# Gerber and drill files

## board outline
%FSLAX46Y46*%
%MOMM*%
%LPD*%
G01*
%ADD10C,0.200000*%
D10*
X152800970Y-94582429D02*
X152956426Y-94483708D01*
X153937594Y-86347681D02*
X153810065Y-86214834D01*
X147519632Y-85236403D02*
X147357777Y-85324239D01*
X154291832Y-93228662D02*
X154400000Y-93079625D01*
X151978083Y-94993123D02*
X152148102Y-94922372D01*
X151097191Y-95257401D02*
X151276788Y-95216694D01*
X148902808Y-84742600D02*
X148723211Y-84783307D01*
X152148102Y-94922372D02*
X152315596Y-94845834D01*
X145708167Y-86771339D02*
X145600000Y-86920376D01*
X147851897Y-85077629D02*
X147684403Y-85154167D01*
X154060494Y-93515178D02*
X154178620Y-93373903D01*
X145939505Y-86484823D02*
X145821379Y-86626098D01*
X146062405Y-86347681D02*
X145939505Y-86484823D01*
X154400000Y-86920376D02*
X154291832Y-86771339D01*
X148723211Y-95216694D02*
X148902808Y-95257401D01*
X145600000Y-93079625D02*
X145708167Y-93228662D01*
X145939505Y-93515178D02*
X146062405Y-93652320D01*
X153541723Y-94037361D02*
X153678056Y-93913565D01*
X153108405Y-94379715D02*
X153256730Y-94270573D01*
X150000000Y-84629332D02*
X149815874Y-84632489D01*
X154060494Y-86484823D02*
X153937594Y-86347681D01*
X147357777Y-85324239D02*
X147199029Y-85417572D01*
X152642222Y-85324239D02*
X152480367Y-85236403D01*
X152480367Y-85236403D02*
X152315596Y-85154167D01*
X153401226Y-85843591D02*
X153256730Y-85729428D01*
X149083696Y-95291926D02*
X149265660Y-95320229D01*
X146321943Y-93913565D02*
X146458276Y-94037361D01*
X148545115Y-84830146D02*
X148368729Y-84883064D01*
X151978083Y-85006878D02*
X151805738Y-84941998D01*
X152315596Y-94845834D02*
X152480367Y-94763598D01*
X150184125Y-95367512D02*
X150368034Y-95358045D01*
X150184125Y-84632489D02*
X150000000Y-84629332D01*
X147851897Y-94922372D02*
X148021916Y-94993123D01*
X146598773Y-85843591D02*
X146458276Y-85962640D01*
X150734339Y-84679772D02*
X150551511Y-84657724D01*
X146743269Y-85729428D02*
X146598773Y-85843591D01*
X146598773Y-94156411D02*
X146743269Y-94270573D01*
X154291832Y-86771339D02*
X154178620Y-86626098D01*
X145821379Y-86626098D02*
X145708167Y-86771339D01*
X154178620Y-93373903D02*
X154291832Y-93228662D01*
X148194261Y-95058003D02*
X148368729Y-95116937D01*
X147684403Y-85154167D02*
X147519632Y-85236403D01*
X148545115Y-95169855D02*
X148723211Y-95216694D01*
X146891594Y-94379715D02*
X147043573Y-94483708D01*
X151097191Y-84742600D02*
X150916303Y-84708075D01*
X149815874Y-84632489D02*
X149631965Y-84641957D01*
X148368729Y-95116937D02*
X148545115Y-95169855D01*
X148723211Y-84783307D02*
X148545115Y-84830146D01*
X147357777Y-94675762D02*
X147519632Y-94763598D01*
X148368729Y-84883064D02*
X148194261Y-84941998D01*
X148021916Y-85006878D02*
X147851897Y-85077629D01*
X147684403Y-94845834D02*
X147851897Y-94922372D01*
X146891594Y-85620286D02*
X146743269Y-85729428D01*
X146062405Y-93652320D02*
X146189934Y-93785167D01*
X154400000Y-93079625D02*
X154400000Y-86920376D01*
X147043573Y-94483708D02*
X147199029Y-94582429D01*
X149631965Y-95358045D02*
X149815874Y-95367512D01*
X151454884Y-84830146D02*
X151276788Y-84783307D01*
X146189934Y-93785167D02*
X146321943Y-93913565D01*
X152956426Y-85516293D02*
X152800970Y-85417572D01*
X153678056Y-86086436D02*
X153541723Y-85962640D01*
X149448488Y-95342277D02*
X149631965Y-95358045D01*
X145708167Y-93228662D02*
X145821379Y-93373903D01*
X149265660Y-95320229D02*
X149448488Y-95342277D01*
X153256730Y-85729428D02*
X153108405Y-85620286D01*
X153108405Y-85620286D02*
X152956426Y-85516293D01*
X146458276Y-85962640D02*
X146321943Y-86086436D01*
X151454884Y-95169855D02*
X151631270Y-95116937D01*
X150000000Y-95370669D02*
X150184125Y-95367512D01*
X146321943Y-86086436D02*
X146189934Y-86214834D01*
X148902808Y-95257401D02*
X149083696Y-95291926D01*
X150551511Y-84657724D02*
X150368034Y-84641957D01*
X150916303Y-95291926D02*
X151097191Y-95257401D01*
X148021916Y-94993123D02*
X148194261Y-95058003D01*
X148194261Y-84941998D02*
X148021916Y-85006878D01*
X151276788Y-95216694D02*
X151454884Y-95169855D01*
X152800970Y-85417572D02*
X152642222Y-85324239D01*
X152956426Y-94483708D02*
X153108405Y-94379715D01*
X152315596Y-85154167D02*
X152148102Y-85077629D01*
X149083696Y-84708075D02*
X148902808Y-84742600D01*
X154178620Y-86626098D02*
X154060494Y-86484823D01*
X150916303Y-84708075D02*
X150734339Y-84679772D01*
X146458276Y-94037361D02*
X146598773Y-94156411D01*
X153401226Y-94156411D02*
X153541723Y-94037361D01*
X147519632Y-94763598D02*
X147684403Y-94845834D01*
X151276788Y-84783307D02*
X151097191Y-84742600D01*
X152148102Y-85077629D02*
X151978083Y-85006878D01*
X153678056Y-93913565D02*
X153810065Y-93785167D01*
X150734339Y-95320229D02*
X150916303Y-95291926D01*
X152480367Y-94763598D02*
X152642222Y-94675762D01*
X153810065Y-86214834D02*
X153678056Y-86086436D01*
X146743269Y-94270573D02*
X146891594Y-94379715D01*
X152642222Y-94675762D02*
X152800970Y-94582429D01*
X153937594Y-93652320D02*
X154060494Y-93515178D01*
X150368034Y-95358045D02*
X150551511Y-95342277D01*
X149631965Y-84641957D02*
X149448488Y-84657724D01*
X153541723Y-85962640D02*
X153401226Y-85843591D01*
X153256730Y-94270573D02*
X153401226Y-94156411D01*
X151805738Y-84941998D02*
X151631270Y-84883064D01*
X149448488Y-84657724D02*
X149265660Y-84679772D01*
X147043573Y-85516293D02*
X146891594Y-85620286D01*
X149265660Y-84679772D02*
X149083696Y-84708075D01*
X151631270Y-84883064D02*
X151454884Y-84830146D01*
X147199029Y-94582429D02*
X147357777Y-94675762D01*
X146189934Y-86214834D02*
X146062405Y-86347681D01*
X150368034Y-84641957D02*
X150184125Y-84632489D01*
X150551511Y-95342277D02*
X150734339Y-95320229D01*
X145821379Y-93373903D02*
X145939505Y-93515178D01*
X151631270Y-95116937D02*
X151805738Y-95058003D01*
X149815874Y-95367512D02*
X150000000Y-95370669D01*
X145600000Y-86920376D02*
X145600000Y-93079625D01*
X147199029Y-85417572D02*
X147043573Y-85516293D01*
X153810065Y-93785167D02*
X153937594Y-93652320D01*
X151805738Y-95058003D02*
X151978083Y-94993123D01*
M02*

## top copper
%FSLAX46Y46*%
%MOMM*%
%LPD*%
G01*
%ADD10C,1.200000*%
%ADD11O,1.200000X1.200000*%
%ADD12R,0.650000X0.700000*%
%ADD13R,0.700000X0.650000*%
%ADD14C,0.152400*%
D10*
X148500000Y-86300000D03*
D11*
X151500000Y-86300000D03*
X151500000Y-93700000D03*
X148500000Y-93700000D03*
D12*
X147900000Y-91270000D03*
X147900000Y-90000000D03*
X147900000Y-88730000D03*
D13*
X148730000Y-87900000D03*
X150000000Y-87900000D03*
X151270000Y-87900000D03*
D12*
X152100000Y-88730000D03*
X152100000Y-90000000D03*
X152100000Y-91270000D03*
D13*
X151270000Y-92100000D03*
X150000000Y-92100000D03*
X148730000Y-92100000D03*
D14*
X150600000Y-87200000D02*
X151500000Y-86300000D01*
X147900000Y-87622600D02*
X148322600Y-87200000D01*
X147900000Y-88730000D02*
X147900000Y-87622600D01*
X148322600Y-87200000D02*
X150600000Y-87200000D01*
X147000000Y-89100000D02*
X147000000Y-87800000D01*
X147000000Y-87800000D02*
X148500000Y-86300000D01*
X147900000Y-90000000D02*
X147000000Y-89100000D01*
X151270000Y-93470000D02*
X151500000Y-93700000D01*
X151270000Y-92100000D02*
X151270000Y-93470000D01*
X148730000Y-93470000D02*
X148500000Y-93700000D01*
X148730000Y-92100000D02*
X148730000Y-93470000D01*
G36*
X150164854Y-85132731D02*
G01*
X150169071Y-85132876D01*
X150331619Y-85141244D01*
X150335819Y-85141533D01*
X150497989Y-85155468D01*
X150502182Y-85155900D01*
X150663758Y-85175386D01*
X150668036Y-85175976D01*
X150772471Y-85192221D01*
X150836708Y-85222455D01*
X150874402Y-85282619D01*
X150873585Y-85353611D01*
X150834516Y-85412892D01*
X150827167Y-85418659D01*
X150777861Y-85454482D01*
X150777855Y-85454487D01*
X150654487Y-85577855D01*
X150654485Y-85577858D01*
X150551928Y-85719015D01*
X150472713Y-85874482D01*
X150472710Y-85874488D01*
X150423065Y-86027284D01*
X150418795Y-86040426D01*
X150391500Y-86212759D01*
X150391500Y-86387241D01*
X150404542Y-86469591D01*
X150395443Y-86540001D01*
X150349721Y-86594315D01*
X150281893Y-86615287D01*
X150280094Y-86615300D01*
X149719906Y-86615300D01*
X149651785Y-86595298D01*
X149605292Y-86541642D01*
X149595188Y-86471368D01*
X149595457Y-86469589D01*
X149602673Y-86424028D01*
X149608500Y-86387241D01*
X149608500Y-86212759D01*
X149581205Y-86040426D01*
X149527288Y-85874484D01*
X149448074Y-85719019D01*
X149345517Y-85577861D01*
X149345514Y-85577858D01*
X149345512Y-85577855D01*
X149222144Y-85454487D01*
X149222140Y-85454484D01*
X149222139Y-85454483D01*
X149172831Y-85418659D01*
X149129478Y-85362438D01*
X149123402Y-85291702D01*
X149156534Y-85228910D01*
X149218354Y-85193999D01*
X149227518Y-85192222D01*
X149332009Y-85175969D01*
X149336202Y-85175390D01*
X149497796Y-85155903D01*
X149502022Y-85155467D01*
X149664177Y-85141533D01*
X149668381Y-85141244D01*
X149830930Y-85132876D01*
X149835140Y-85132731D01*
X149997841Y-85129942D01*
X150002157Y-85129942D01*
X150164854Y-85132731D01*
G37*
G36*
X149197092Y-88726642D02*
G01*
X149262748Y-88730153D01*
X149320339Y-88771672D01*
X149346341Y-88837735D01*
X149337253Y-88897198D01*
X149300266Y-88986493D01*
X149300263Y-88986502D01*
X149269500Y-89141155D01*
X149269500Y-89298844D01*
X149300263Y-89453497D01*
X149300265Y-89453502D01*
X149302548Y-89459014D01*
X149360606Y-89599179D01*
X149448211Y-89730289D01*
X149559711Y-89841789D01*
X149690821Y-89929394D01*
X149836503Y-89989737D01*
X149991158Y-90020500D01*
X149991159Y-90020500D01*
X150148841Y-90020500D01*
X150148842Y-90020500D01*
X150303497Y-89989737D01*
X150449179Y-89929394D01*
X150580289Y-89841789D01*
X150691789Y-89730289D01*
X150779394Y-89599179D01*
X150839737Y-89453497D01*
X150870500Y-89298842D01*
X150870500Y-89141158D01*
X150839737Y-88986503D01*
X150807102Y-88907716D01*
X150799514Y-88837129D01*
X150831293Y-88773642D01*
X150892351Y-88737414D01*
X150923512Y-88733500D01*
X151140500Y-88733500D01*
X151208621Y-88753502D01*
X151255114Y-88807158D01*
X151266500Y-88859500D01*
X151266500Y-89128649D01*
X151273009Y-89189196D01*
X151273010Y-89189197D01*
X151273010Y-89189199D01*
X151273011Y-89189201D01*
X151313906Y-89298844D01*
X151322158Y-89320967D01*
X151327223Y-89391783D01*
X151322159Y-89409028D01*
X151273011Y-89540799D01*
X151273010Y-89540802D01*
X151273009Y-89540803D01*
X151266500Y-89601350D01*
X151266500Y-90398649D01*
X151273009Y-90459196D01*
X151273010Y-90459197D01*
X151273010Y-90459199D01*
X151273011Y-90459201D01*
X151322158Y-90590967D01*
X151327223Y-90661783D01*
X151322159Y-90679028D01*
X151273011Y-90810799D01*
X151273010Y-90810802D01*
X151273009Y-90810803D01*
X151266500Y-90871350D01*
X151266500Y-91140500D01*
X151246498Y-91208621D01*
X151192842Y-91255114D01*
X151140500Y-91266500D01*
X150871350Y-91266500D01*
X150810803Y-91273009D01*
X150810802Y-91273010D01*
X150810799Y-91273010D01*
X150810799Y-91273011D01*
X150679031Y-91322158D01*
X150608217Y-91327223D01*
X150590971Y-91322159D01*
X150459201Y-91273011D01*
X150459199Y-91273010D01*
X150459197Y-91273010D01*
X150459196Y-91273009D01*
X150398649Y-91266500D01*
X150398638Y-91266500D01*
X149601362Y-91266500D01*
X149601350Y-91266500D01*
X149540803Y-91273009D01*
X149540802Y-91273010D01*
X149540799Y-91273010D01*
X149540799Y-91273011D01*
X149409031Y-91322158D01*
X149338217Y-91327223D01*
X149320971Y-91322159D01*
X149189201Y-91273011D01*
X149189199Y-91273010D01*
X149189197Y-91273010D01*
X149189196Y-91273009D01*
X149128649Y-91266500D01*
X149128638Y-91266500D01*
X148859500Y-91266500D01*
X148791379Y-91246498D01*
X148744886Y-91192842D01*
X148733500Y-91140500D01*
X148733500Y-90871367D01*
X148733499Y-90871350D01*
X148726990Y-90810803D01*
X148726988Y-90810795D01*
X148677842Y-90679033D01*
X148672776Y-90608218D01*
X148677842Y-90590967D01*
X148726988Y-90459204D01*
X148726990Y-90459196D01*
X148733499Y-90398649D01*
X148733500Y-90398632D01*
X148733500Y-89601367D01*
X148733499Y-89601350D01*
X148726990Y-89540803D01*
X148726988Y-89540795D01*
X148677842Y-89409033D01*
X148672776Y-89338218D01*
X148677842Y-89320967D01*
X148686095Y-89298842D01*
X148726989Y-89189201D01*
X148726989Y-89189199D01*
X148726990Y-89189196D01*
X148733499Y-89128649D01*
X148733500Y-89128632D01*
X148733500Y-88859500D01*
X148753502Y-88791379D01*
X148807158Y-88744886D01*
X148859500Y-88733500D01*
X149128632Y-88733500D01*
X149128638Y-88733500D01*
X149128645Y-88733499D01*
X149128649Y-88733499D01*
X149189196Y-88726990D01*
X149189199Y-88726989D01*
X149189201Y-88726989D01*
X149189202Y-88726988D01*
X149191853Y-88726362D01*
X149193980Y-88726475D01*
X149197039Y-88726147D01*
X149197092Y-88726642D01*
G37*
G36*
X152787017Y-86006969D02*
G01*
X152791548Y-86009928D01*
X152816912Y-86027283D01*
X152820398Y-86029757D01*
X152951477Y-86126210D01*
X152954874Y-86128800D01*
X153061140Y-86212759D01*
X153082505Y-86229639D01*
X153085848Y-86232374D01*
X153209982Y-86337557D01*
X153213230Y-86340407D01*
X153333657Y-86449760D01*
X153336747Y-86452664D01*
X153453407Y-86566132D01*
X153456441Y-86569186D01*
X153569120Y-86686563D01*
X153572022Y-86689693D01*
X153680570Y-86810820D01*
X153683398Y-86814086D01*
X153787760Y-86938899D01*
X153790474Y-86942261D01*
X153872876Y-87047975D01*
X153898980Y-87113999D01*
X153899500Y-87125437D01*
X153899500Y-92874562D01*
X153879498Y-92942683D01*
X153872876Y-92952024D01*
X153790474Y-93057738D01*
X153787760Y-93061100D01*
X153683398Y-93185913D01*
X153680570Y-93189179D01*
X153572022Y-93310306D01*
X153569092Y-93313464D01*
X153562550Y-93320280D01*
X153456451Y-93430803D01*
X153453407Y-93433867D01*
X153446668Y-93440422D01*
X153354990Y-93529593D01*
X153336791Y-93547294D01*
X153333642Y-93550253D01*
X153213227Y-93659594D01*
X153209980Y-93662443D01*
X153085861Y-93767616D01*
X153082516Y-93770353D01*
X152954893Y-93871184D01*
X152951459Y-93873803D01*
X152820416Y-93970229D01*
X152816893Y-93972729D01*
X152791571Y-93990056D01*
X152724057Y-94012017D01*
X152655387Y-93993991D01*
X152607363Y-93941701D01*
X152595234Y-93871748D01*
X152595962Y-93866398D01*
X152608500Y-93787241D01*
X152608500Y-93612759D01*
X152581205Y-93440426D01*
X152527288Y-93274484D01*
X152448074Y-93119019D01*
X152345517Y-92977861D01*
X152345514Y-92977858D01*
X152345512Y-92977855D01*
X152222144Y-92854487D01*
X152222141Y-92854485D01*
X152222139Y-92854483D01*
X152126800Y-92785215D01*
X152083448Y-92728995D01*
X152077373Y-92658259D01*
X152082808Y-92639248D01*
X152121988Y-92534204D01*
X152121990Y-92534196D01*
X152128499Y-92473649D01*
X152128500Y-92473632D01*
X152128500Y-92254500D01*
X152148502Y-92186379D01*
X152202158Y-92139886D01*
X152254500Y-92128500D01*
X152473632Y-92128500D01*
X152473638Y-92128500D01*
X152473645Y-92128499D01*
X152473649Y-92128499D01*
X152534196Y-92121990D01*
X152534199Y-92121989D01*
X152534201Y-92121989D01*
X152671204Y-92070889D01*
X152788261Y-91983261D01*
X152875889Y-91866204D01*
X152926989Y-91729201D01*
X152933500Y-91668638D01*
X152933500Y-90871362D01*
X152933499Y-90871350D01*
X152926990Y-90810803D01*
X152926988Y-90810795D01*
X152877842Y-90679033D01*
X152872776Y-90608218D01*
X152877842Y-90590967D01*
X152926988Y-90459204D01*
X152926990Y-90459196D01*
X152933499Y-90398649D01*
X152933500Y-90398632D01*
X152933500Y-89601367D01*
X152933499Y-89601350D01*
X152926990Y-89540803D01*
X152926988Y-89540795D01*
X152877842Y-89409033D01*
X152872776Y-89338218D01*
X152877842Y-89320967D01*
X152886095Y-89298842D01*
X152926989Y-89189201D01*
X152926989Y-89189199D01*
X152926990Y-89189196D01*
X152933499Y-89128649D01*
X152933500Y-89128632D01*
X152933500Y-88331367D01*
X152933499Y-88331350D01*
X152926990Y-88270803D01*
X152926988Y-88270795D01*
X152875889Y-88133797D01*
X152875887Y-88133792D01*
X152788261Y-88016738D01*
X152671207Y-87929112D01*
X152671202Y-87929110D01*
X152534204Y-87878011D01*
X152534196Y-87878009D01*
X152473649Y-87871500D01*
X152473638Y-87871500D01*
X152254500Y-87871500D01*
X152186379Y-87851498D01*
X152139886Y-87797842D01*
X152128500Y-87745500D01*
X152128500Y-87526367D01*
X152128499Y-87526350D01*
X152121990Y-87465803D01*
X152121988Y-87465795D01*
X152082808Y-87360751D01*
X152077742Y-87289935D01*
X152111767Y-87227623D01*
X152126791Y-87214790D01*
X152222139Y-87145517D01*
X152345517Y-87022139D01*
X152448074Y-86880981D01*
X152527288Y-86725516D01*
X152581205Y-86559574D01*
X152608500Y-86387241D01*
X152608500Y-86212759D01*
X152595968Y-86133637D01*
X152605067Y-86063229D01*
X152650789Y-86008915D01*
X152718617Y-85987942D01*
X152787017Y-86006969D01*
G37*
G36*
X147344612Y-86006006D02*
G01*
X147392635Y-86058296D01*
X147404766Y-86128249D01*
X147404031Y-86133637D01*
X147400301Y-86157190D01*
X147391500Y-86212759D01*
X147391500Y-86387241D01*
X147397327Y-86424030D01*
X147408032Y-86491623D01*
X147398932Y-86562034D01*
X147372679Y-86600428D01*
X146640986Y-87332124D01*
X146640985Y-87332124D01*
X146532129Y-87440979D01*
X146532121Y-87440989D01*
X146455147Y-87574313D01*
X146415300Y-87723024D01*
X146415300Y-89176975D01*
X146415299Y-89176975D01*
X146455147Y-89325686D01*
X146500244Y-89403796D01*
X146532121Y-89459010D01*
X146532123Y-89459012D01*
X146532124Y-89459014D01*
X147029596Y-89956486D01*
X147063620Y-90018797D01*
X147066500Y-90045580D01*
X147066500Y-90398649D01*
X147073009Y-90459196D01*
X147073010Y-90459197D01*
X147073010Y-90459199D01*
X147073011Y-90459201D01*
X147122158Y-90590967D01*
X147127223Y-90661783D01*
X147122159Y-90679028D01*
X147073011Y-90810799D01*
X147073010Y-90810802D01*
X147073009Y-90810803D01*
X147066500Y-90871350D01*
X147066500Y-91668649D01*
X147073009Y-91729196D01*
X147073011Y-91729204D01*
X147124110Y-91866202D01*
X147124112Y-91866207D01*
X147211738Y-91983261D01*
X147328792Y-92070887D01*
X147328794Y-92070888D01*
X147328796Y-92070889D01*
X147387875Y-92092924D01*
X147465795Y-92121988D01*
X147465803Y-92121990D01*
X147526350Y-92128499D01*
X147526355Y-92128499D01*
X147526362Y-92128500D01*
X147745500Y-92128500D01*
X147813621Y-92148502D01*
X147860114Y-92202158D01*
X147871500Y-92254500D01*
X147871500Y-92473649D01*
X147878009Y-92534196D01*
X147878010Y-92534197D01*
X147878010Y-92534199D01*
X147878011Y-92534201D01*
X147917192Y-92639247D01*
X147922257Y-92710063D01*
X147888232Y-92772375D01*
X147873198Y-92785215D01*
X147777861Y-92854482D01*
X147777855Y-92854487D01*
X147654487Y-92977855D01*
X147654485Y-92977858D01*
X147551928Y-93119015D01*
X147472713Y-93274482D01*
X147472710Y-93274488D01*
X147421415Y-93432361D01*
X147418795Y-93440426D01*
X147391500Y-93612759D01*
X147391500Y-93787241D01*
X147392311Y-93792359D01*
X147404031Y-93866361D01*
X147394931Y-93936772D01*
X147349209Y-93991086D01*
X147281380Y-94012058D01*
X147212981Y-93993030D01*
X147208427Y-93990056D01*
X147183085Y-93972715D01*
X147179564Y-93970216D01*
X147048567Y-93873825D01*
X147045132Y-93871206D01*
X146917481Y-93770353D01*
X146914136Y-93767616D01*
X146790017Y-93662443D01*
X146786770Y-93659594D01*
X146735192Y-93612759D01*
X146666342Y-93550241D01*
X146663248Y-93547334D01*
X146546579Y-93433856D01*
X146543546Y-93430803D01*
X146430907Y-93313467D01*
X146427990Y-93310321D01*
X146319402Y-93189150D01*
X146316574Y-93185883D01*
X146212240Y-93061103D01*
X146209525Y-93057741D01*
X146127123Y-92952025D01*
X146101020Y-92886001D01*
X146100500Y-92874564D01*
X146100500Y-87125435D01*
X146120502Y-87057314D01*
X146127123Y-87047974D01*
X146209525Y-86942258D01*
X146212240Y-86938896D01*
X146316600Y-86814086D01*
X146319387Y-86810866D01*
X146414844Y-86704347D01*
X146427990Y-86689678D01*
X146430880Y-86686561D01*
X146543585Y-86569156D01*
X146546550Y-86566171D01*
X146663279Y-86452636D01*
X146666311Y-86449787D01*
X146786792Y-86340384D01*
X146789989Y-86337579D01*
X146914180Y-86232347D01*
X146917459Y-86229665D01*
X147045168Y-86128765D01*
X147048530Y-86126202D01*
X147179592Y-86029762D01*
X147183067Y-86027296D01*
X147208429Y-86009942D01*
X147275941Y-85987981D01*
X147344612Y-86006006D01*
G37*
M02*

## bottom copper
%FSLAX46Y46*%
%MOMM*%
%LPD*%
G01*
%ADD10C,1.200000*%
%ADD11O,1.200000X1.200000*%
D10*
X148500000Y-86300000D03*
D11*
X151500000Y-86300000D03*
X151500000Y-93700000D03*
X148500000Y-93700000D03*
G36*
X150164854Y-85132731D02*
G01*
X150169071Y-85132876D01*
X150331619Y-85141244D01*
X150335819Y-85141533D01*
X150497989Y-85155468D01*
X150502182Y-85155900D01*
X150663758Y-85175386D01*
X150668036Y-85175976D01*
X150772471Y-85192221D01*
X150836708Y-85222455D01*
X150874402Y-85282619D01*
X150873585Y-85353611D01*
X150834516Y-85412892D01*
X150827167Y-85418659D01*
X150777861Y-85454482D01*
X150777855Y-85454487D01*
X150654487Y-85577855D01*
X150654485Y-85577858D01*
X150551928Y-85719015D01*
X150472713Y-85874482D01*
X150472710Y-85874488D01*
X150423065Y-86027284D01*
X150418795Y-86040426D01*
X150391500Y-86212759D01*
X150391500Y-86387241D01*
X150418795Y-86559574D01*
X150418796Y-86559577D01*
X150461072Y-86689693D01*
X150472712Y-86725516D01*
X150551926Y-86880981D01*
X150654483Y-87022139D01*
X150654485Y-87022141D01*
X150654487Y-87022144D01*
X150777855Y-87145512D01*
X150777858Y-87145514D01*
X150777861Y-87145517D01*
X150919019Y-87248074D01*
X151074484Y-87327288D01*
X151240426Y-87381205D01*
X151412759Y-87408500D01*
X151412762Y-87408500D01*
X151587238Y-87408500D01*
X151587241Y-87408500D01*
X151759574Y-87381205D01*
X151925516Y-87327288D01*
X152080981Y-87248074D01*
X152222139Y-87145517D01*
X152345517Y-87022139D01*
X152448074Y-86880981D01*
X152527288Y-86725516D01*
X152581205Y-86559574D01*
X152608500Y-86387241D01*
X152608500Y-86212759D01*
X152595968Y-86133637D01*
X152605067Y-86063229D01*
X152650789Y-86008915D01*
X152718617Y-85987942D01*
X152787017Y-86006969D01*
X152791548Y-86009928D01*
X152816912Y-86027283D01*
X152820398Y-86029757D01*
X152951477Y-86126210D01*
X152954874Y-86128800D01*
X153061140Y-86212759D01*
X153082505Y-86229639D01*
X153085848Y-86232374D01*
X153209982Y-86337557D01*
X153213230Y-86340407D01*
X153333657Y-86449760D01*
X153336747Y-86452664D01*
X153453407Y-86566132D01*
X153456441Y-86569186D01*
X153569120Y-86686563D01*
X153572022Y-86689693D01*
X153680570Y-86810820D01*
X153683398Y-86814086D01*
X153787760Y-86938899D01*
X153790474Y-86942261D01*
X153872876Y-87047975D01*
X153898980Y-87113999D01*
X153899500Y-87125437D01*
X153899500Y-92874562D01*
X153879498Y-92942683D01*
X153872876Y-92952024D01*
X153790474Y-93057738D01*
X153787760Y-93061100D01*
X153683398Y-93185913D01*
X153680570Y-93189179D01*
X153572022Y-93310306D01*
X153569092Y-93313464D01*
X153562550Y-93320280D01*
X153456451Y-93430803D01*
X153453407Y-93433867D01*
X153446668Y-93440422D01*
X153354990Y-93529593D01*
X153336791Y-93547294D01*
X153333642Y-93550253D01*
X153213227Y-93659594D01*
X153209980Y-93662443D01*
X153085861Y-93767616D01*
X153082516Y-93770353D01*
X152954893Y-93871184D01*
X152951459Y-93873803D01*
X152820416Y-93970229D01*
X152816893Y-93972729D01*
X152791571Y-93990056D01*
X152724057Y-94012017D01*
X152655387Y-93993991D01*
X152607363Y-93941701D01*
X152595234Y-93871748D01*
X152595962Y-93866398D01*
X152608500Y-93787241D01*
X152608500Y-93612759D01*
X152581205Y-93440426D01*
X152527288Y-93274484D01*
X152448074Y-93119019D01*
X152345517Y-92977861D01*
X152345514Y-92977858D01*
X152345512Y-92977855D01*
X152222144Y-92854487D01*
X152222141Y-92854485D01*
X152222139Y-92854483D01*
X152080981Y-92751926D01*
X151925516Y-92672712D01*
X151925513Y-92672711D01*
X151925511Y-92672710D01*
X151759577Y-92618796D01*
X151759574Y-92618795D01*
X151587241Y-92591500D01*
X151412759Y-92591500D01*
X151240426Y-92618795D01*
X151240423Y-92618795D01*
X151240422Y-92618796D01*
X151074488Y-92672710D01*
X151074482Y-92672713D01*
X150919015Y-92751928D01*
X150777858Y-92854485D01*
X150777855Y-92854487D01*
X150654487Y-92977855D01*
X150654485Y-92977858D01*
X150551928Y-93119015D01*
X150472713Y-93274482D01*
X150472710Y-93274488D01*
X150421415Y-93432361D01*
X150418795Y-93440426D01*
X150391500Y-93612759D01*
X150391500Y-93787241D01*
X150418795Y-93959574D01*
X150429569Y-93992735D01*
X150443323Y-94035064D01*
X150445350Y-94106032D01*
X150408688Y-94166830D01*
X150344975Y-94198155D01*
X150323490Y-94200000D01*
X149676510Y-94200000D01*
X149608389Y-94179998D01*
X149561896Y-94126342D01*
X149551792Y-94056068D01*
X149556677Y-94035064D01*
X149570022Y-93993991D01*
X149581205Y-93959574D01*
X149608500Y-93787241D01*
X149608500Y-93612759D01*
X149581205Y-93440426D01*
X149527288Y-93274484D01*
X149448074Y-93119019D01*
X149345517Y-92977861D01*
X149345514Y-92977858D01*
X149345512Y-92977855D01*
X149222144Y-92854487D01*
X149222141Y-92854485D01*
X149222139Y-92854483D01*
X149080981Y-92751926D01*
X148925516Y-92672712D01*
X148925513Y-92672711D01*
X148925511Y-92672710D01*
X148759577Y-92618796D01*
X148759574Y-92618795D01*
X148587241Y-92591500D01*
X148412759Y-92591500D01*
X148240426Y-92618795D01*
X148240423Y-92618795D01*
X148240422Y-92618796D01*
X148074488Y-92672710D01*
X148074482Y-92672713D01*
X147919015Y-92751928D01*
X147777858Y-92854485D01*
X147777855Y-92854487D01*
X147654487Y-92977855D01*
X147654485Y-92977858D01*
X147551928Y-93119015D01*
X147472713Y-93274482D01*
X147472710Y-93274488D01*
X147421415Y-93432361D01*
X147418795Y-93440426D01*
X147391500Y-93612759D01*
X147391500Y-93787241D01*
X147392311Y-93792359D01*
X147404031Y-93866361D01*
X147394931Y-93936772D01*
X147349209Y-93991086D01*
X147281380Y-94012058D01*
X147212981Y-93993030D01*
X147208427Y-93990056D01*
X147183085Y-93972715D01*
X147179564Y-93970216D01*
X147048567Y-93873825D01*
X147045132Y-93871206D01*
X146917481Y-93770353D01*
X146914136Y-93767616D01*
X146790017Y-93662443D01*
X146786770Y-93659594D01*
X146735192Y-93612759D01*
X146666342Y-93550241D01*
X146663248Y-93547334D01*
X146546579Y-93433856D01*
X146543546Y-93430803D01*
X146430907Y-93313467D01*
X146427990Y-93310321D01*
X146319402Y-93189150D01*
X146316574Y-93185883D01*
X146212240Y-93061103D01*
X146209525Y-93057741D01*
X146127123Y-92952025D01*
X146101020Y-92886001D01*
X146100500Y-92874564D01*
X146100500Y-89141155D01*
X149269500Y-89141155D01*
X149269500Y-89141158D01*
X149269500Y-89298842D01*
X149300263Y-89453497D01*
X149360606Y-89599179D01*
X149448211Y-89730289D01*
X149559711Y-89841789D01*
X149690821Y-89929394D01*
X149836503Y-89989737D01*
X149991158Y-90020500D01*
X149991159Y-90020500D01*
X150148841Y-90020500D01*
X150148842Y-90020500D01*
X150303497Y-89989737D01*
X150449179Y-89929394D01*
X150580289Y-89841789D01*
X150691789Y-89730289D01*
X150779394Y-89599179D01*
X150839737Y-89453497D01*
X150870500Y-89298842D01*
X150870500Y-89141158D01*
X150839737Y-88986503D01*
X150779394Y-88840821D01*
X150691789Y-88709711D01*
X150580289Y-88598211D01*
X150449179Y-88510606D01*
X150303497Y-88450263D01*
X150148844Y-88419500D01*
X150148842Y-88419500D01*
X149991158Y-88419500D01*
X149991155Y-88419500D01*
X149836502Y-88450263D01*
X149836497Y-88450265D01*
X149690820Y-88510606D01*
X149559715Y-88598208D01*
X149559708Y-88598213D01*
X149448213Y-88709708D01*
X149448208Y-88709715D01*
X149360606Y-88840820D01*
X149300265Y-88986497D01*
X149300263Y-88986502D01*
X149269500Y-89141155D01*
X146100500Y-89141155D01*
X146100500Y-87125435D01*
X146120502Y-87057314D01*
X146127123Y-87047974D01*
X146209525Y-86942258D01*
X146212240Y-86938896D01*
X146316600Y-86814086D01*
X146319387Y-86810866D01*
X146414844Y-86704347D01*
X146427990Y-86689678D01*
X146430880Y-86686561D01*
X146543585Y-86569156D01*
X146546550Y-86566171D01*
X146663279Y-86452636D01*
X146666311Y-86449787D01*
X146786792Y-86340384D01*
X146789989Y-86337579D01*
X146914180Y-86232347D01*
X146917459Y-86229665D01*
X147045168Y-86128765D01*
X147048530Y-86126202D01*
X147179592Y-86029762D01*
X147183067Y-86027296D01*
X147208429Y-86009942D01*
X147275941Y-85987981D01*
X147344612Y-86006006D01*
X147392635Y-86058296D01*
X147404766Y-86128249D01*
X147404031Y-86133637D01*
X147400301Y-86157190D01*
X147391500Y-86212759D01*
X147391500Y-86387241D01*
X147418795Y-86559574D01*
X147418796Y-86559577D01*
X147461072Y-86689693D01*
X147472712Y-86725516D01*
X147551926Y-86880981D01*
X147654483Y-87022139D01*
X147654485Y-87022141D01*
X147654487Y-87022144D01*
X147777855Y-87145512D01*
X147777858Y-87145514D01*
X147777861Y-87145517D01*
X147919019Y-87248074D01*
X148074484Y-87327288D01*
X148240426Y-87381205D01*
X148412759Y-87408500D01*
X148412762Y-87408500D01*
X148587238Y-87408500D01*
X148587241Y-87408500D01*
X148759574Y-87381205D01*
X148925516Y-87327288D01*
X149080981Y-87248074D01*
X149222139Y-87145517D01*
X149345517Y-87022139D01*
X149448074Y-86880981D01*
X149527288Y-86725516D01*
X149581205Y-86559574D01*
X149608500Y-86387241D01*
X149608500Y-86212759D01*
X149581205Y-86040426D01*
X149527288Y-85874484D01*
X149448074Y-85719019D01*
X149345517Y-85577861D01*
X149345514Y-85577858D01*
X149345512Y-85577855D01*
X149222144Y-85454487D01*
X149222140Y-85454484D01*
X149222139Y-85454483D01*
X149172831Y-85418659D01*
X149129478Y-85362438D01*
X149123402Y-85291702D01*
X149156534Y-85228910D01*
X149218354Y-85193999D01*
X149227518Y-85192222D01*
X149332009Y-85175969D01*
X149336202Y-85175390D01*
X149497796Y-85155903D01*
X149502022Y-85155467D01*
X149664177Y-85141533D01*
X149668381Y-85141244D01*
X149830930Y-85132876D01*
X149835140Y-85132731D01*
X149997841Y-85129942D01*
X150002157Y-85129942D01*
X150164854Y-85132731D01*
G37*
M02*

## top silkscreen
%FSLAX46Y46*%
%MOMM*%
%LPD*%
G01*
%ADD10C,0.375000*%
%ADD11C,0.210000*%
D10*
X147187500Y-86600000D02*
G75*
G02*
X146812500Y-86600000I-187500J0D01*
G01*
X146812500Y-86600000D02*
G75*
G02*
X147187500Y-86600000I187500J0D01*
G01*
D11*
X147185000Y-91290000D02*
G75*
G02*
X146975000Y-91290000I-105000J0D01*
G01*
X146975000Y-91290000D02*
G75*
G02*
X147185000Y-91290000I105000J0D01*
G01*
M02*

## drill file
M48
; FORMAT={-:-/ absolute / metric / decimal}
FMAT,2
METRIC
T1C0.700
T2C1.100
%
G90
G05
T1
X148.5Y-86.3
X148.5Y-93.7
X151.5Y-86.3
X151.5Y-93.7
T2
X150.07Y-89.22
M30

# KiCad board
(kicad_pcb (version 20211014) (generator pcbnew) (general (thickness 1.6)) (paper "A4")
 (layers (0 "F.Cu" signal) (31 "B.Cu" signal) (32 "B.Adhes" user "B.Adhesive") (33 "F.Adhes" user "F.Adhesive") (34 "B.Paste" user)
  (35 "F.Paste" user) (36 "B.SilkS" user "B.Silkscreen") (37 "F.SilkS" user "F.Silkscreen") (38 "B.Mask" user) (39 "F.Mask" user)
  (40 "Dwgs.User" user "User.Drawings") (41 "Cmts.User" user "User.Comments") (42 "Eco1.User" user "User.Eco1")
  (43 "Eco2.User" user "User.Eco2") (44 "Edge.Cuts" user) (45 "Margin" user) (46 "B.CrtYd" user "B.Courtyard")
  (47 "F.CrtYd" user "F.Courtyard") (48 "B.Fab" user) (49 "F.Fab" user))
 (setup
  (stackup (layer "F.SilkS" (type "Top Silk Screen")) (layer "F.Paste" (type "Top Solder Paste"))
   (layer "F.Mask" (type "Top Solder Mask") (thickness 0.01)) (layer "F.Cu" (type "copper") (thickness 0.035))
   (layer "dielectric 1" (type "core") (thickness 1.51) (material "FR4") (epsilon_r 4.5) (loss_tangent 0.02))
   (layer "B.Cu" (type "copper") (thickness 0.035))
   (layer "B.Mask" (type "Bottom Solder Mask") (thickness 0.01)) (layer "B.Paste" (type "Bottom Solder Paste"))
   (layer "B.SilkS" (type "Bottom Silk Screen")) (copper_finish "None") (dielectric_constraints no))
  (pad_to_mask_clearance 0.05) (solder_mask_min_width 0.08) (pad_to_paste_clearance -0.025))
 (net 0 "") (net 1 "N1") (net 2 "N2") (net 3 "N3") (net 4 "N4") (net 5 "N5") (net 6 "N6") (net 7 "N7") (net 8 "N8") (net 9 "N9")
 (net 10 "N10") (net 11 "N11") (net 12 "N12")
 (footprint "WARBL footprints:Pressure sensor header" (layer "F.Cu") (at 148.5 86.3)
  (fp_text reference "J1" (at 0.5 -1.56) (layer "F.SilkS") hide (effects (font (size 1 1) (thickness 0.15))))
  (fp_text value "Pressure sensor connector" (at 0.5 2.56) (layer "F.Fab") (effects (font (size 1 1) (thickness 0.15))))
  (pad "1" thru_hole circle (at 0 0) (size 1.2 1.2) (drill 0.7) (layers *.Cu *.Mask) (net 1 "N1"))
  (pad "2" thru_hole oval (at 3 0) (size 1.2 1.2) (drill 0.7) (layers *.Cu *.Mask) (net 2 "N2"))
  (pad "3" thru_hole oval (at 3 7.4) (size 1.2 1.2) (drill 0.7) (layers *.Cu *.Mask) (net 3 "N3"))
  (pad "4" thru_hole oval (at 0 7.4) (size 1.2 1.2) (drill 0.7) (layers *.Cu *.Mask) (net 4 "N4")))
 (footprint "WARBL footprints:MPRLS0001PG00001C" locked (layer "F.Cu") (at 150 90 -90)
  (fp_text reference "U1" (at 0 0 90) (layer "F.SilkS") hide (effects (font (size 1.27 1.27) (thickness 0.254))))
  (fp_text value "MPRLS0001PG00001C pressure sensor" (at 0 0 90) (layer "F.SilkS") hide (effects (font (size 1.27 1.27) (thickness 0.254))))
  (fp_circle (center 1.29 2.92) (end 1.44 2.92) (layer "F.SilkS") (width 0.12) (fill solid))
  (pad "" np_thru_hole circle locked (at -0.78 -0.07 270) (size 1.1 1.1) (drill 1.1) (layers *.Cu *.Mask))
  (pad "1" smd rect locked (at 1.27 2.1) (size 0.65 0.7) (layers "F.Cu" "F.Paste" "F.Mask") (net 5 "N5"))
  (pad "2" smd rect locked (at 0 2.1) (size 0.65 0.7) (layers "F.Cu" "F.Paste" "F.Mask") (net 1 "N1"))
  (pad "3" smd rect locked (at -1.27 2.1) (size 0.65 0.7) (layers "F.Cu" "F.Paste" "F.Mask") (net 2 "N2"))
  (pad "4" smd rect locked (at -2.1 1.27 270) (size 0.65 0.7) (layers "F.Cu" "F.Paste" "F.Mask") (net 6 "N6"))
  (pad "5" smd rect locked (at -2.1 0 270) (size 0.65 0.7) (layers "F.Cu" "F.Paste" "F.Mask") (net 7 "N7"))
  (pad "6" smd rect locked (at -2.1 -1.27 270) (size 0.65 0.7) (layers "F.Cu" "F.Paste" "F.Mask") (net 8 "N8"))
  (pad "7" smd rect locked (at -1.27 -2.1) (size 0.65 0.7) (layers "F.Cu" "F.Paste" "F.Mask") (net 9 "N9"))
  (pad "8" smd rect locked (at 0 -2.1) (size 0.65 0.7) (layers "F.Cu" "F.Paste" "F.Mask") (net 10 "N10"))
  (pad "9" smd rect locked (at 1.27 -2.1) (size 0.65 0.7) (layers "F.Cu" "F.Paste" "F.Mask") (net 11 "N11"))
  (pad "10" smd rect locked (at 2.1 -1.27 270) (size 0.65 0.7) (layers "F.Cu" "F.Paste" "F.Mask") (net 3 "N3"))
  (pad "11" smd rect locked (at 2.1 0 270) (size 0.65 0.7) (layers "F.Cu" "F.Paste" "F.Mask") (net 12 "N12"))
  (pad "12" smd rect locked (at 2.1 1.27 270) (size 0.65 0.7) (layers "F.Cu" "F.Paste" "F.Mask") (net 4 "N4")))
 (gr_circle (center 147 86.6) (end 147.3 86.6) (layer "F.SilkS") (width 0.15) (fill solid))
 (gr_line locked (start 152.80097 94.582429) (end 152.956426 94.483708) (layer "Edge.Cuts") (width 0.2))
 (gr_line locked (start 153.937594 86.347681) (end 153.810065 86.214834) (layer "Edge.Cuts") (width 0.2))
 (gr_line locked (start 147.519632 85.236403) (end 147.357777 85.324239) (layer "Edge.Cuts") (width 0.2))
 (gr_line locked (start 154.291832 93.228662) (end 154.4 93.079625) (layer "Edge.Cuts") (width 0.2))
 (gr_line locked (start 151.978083 94.993123) (end 152.148102 94.922372) (layer "Edge.Cuts") (width 0.2))
 (gr_line locked (start 151.097191 95.257401) (end 151.276788 95.216694) (layer "Edge.Cuts") (width 0.2))
 (gr_line locked (start 148.902808 84.7426) (end 148.723211 84.783307) (layer "Edge.Cuts") (width 0.2))
 (gr_line locked (start 152.148102 94.922372) (end 152.315596 94.845834) (layer "Edge.Cuts") (width 0.2))
 (gr_line locked (start 145.708167 86.771339) (end 145.6 86.920376) (layer "Edge.Cuts") (width 0.2))
 (gr_line locked (start 147.851897 85.077629) (end 147.684403 85.154167) (layer "Edge.Cuts") (width 0.2))
 (gr_line locked (start 154.060494 93.515178) (end 154.17862 93.373903) (layer "Edge.Cuts") (width 0.2))
 (gr_line locked (start 145.939505 86.484823) (end 145.821379 86.626098) (layer "Edge.Cuts") (width 0.2))
 (gr_line locked (start 146.062405 86.347681) (end 145.939505 86.484823) (layer "Edge.Cuts") (width 0.2))
 (gr_line locked (start 154.4 86.920376) (end 154.291832 86.771339) (layer "Edge.Cuts") (width 0.2))
 (gr_line locked (start 148.723211 95.216694) (end 148.902808 95.257401) (layer "Edge.Cuts") (width 0.2))
 (gr_line locked (start 145.6 93.079625) (end 145.708167 93.228662) (layer "Edge.Cuts") (width 0.2))
 (gr_line locked (start 145.939505 93.515178) (end 146.062405 93.65232) (layer "Edge.Cuts") (width 0.2))
 (gr_line locked (start 153.541723 94.037361) (end 153.678056 93.913565) (layer "Edge.Cuts") (width 0.2))
 (gr_line locked (start 153.108405 94.379715) (end 153.25673 94.270573) (layer "Edge.Cuts") (width 0.2))
 (gr_line locked (start 150 84.629332) (end 149.815874 84.632489) (layer "Edge.Cuts") (width 0.2))
 (gr_line locked (start 154.060494 86.484823) (end 153.937594 86.347681) (layer "Edge.Cuts") (width 0.2))
 (gr_line locked (start 147.357777 85.324239) (end 147.199029 85.417572) (layer "Edge.Cuts") (width 0.2))
 (gr_line locked (start 152.642222 85.324239) (end 152.480367 85.236403) (layer "Edge.Cuts") (width 0.2))
 (gr_line locked (start 152.480367 85.236403) (end 152.315596 85.154167) (layer "Edge.Cuts") (width 0.2))
 (gr_line locked (start 153.401226 85.843591) (end 153.25673 85.729428) (layer "Edge.Cuts") (width 0.2))
 (gr_line locked (start 149.083696 95.291926) (end 149.26566 95.320229) (layer "Edge.Cuts") (width 0.2))
 (gr_line locked (start 146.321943 93.913565) (end 146.458276 94.037361) (layer "Edge.Cuts") (width 0.2))
 (gr_line locked (start 148.545115 84.830146) (end 148.368729 84.883064) (layer "Edge.Cuts") (width 0.2))
 (gr_line locked (start 151.978083 85.006878) (end 151.805738 84.941998) (layer "Edge.Cuts") (width 0.2))
 (gr_line locked (start 152.315596 94.845834) (end 152.480367 94.763598) (layer "Edge.Cuts") (width 0.2))
 (gr_line locked (start 150.184125 95.367512) (end 150.368034 95.358045) (layer "Edge.Cuts") (width 0.2))
 (gr_line locked (start 150.184125 84.632489) (end 150 84.629332) (layer "Edge.Cuts") (width 0.2))
 (gr_line locked (start 147.851897 94.922372) (end 148.021916 94.993123) (layer "Edge.Cuts") (width 0.2))
 (gr_line locked (start 146.598773 85.843591) (end 146.458276 85.96264) (layer "Edge.Cuts") (width 0.2))
 (gr_line locked (start 150.734339 84.679772) (end 150.551511 84.657724) (layer "Edge.Cuts") (width 0.2))
 (gr_line locked (start 146.743269 85.729428) (end 146.598773 85.843591) (layer "Edge.Cuts") (width 0.2))
 (gr_line locked (start 146.598773 94.156411) (end 146.743269 94.270573) (layer "Edge.Cuts") (width 0.2))
 (gr_line locked (start 154.291832 86.771339) (end 154.17862 86.626098) (layer "Edge.Cuts") (width 0.2))
 (gr_line locked (start 145.821379 86.626098) (end 145.708167 86.771339) (layer "Edge.Cuts") (width 0.2))
 (gr_line locked (start 154.17862 93.373903) (end 154.291832 93.228662) (layer "Edge.Cuts") (width 0.2))
 (gr_line locked (start 148.194261 95.058003) (end 148.368729 95.116937) (layer "Edge.Cuts") (width 0.2))
 (gr_line locked (start 147.684403 85.154167) (end 147.519632 85.236403) (layer "Edge.Cuts") (width 0.2))
 (gr_line locked (start 148.545115 95.169855) (end 148.723211 95.216694) (layer "Edge.Cuts") (width 0.2))
 (gr_line locked (start 146.891594 94.379715) (end 147.043573 94.483708) (layer "Edge.Cuts") (width 0.2))
 (gr_line locked (start 151.097191 84.7426) (end 150.916303 84.708075) (layer "Edge.Cuts") (width 0.2))
 (gr_line locked (start 149.815874 84.632489) (end 149.631965 84.641957) (layer "Edge.Cuts") (width 0.2))
 (gr_line locked (start 148.368729 95.116937) (end 148.545115 95.169855) (layer "Edge.Cuts") (width 0.2))
 (gr_line locked (start 148.723211 84.783307) (end 148.545115 84.830146) (layer "Edge.Cuts") (width 0.2))
 (gr_line locked (start 147.357777 94.675762) (end 147.519632 94.763598) (layer "Edge.Cuts") (width 0.2))
 (gr_line locked (start 148.368729 84.883064) (end 148.194261 84.941998) (layer "Edge.Cuts") (width 0.2))
 (gr_line locked (start 148.021916 85.006878) (end 147.851897 85.077629) (layer "Edge.Cuts") (width 0.2))
 (gr_line locked (start 147.684403 94.845834) (end 147.851897 94.922372) (layer "Edge.Cuts") (width 0.2))
 (gr_line locked (start 146.891594 85.620286) (end 146.743269 85.729428) (layer "Edge.Cuts") (width 0.2))
 (gr_line locked (start 146.062405 93.65232) (end 146.189934 93.785167) (layer "Edge.Cuts") (width 0.2))
 (gr_line locked (start 154.4 93.079625) (end 154.4 86.920376) (layer "Edge.Cuts") (width 0.2))
 (gr_line locked (start 147.043573 94.483708) (end 147.199029 94.582429) (layer "Edge.Cuts") (width 0.2))
 (gr_line locked (start 149.631965 95.358045) (end 149.815874 95.367512) (layer "Edge.Cuts") (width 0.2))
 (gr_line locked (start 151.454884 84.830146) (end 151.276788 84.783307) (layer "Edge.Cuts") (width 0.2))
 (gr_line locked (start 146.189934 93.785167) (end 146.321943 93.913565) (layer "Edge.Cuts") (width 0.2))
 (gr_line locked (start 152.956426 85.516293) (end 152.80097 85.417572) (layer "Edge.Cuts") (width 0.2))
 (gr_line locked (start 153.678056 86.086436) (end 153.541723 85.96264) (layer "Edge.Cuts") (width 0.2))
 (gr_line locked (start 149.448488 95.342277) (end 149.631965 95.358045) (layer "Edge.Cuts") (width 0.2))
 (gr_line locked (start 145.708167 93.228662) (end 145.821379 93.373903) (layer "Edge.Cuts") (width 0.2))
 (gr_line locked (start 149.26566 95.320229) (end 149.448488 95.342277) (layer "Edge.Cuts") (width 0.2))
 (gr_line locked (start 153.25673 85.729428) (end 153.108405 85.620286) (layer "Edge.Cuts") (width 0.2))
 (gr_line locked (start 153.108405 85.620286) (end 152.956426 85.516293) (layer "Edge.Cuts") (width 0.2))
 (gr_line locked (start 146.458276 85.96264) (end 146.321943 86.086436) (layer "Edge.Cuts") (width 0.2))
 (gr_line locked (start 151.454884 95.169855) (end 151.63127 95.116937) (layer "Edge.Cuts") (width 0.2))
 (gr_line locked (start 150 95.370669) (end 150.184125 95.367512) (layer "Edge.Cuts") (width 0.2))
 (gr_line locked (start 146.321943 86.086436) (end 146.189934 86.214834) (layer "Edge.Cuts") (width 0.2))
 (gr_line locked (start 148.902808 95.257401) (end 149.083696 95.291926) (layer "Edge.Cuts") (width 0.2))
 (gr_line locked (start 150.551511 84.657724) (end 150.368034 84.641957) (layer "Edge.Cuts") (width 0.2))
 (gr_line locked (start 150.916303 95.291926) (end 151.097191 95.257401) (layer "Edge.Cuts") (width 0.2))
 (gr_line locked (start 148.021916 94.993123) (end 148.194261 95.058003) (layer "Edge.Cuts") (width 0.2))
 (gr_line locked (start 148.194261 84.941998) (end 148.021916 85.006878) (layer "Edge.Cuts") (width 0.2))
 (gr_line locked (start 151.276788 95.216694) (end 151.454884 95.169855) (layer "Edge.Cuts") (width 0.2))
 (gr_line locked (start 152.80097 85.417572) (end 152.642222 85.324239) (layer "Edge.Cuts") (width 0.2))
 (gr_line locked (start 152.956426 94.483708) (end 153.108405 94.379715) (layer "Edge.Cuts") (width 0.2))
 (gr_line locked (start 152.315596 85.154167) (end 152.148102 85.077629) (layer "Edge.Cuts") (width 0.2))
 (gr_line locked (start 149.083696 84.708075) (end 148.902808 84.7426) (layer "Edge.Cuts") (width 0.2))
 (gr_line locked (start 154.17862 86.626098) (end 154.060494 86.484823) (layer "Edge.Cuts") (width 0.2))
 (gr_line locked (start 150.916303 84.708075) (end 150.734339 84.679772) (layer "Edge.Cuts") (width 0.2))
 (gr_line locked (start 146.458276 94.037361) (end 146.598773 94.156411) (layer "Edge.Cuts") (width 0.2))
 (gr_line locked (start 153.401226 94.156411) (end 153.541723 94.037361) (layer "Edge.Cuts") (width 0.2))
 (gr_line locked (start 147.519632 94.763598) (end 147.684403 94.845834) (layer "Edge.Cuts") (width 0.2))
 (gr_line locked (start 151.276788 84.783307) (end 151.097191 84.7426) (layer "Edge.Cuts") (width 0.2))
 (gr_line locked (start 152.148102 85.077629) (end 151.978083 85.006878) (layer "Edge.Cuts") (width 0.2))
 (gr_line locked (start 153.678056 93.913565) (end 153.810065 93.785167) (layer "Edge.Cuts") (width 0.2))
 (gr_line locked (start 150.734339 95.320229) (end 150.916303 95.291926) (layer "Edge.Cuts") (width 0.2))
 (gr_line locked (start 152.480367 94.763598) (end 152.642222 94.675762) (layer "Edge.Cuts") (width 0.2))
 (gr_line locked (start 153.810065 86.214834) (end 153.678056 86.086436) (layer "Edge.Cuts") (width 0.2))
 (gr_line locked (start 146.743269 94.270573) (end 146.891594 94.379715) (layer "Edge.Cuts") (width 0.2))
 (gr_line locked (start 152.642222 94.675762) (end 152.80097 94.582429) (layer "Edge.Cuts") (width 0.2))
 (gr_line locked (start 153.937594 93.65232) (end 154.060494 93.515178) (layer "Edge.Cuts") (width 0.2))
 (gr_line locked (start 150.368034 95.358045) (end 150.551511 95.342277) (layer "Edge.Cuts") (width 0.2))
 (gr_line locked (start 149.631965 84.641957) (end 149.448488 84.657724) (layer "Edge.Cuts") (width 0.2))
 (gr_line locked (start 153.541723 85.96264) (end 153.401226 85.843591) (layer "Edge.Cuts") (width 0.2))
 (gr_line locked (start 153.25673 94.270573) (end 153.401226 94.156411) (layer "Edge.Cuts") (width 0.2))
 (gr_line locked (start 151.805738 84.941998) (end 151.63127 84.883064) (layer "Edge.Cuts") (width 0.2))
 (gr_line locked (start 149.448488 84.657724) (end 149.26566 84.679772) (layer "Edge.Cuts") (width 0.2))
 (gr_line locked (start 147.043573 85.516293) (end 146.891594 85.620286) (layer "Edge.Cuts") (width 0.2))
 (gr_line locked (start 149.26566 84.679772) (end 149.083696 84.708075) (layer "Edge.Cuts") (width 0.2))
 (gr_line locked (start 151.63127 84.883064) (end 151.454884 84.830146) (layer "Edge.Cuts") (width 0.2))
 (gr_line locked (start 147.199029 94.582429) (end 147.357777 94.675762) (layer "Edge.Cuts") (width 0.2))
 (gr_line locked (start 146.189934 86.214834) (end 146.062405 86.347681) (layer "Edge.Cuts") (width 0.2))
 (gr_line locked (start 150.368034 84.641957) (end 150.184125 84.632489) (layer "Edge.Cuts") (width 0.2))
 (gr_line locked (start 150.551511 95.342277) (end 150.734339 95.320229) (layer "Edge.Cuts") (width 0.2))
 (gr_line locked (start 145.821379 93.373903) (end 145.939505 93.515178) (layer "Edge.Cuts") (width 0.2))
 (gr_line locked (start 151.63127 95.116937) (end 151.805738 95.058003) (layer "Edge.Cuts") (width 0.2))
 (gr_line locked (start 149.815874 95.367512) (end 150 95.370669) (layer "Edge.Cuts") (width 0.2))
 (gr_line locked (start 145.6 86.920376) (end 145.6 93.079625) (layer "Edge.Cuts") (width 0.2))
 (gr_line locked (start 147.199029 85.417572) (end 147.043573 85.516293) (layer "Edge.Cuts") (width 0.2))
 (gr_line locked (start 153.810065 93.785167) (end 153.937594 93.65232) (layer "Edge.Cuts") (width 0.2))
 (gr_line locked (start 151.805738 95.058003) (end 151.978083 94.993123) (layer "Edge.Cuts") (width 0.2))
 (segment (start 150.6 87.2) (end 151.5 86.3) (width 0.1524) (layer "F.Cu") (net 2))
 (segment (start 147.9 87.6226) (end 148.3226 87.2) (width 0.1524) (layer "F.Cu") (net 2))
 (segment (start 147.9 88.73) (end 147.9 87.6226) (width 0.1524) (layer "F.Cu") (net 2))
 (segment (start 148.3226 87.2) (end 150.6 87.2) (width 0.1524) (layer "F.Cu") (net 2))
 (segment (start 147 89.1) (end 147 87.8) (width 0.1524) (layer "F.Cu") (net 1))
 (segment (start 147 87.8) (end 148.5 86.3) (width 0.1524) (layer "F.Cu") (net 1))
 (segment (start 147.9 90) (end 147 89.1) (width 0.1524) (layer "F.Cu") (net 1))
 (segment (start 151.27 93.47) (end 151.5 93.7) (width 0.1524) (layer "F.Cu") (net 3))
 (segment (start 151.27 92.1) (end 151.27 93.47) (width 0.1524) (layer "F.Cu") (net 3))
 (segment (start 148.73 93.47) (end 148.5 93.7) (width 0.1524) (layer "F.Cu") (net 4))
 (segment (start 148.73 92.1) (end 148.73 93.47) (width 0.1524) (layer "F.Cu") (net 4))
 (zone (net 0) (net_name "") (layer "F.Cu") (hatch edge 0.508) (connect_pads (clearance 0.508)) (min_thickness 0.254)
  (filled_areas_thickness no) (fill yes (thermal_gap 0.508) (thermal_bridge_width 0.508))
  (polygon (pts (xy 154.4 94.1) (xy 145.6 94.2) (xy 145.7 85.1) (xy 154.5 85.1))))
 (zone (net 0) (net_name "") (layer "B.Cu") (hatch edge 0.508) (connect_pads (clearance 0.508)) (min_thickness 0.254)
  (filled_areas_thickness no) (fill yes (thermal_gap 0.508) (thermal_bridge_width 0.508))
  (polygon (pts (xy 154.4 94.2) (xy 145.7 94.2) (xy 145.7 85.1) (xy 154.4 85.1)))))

